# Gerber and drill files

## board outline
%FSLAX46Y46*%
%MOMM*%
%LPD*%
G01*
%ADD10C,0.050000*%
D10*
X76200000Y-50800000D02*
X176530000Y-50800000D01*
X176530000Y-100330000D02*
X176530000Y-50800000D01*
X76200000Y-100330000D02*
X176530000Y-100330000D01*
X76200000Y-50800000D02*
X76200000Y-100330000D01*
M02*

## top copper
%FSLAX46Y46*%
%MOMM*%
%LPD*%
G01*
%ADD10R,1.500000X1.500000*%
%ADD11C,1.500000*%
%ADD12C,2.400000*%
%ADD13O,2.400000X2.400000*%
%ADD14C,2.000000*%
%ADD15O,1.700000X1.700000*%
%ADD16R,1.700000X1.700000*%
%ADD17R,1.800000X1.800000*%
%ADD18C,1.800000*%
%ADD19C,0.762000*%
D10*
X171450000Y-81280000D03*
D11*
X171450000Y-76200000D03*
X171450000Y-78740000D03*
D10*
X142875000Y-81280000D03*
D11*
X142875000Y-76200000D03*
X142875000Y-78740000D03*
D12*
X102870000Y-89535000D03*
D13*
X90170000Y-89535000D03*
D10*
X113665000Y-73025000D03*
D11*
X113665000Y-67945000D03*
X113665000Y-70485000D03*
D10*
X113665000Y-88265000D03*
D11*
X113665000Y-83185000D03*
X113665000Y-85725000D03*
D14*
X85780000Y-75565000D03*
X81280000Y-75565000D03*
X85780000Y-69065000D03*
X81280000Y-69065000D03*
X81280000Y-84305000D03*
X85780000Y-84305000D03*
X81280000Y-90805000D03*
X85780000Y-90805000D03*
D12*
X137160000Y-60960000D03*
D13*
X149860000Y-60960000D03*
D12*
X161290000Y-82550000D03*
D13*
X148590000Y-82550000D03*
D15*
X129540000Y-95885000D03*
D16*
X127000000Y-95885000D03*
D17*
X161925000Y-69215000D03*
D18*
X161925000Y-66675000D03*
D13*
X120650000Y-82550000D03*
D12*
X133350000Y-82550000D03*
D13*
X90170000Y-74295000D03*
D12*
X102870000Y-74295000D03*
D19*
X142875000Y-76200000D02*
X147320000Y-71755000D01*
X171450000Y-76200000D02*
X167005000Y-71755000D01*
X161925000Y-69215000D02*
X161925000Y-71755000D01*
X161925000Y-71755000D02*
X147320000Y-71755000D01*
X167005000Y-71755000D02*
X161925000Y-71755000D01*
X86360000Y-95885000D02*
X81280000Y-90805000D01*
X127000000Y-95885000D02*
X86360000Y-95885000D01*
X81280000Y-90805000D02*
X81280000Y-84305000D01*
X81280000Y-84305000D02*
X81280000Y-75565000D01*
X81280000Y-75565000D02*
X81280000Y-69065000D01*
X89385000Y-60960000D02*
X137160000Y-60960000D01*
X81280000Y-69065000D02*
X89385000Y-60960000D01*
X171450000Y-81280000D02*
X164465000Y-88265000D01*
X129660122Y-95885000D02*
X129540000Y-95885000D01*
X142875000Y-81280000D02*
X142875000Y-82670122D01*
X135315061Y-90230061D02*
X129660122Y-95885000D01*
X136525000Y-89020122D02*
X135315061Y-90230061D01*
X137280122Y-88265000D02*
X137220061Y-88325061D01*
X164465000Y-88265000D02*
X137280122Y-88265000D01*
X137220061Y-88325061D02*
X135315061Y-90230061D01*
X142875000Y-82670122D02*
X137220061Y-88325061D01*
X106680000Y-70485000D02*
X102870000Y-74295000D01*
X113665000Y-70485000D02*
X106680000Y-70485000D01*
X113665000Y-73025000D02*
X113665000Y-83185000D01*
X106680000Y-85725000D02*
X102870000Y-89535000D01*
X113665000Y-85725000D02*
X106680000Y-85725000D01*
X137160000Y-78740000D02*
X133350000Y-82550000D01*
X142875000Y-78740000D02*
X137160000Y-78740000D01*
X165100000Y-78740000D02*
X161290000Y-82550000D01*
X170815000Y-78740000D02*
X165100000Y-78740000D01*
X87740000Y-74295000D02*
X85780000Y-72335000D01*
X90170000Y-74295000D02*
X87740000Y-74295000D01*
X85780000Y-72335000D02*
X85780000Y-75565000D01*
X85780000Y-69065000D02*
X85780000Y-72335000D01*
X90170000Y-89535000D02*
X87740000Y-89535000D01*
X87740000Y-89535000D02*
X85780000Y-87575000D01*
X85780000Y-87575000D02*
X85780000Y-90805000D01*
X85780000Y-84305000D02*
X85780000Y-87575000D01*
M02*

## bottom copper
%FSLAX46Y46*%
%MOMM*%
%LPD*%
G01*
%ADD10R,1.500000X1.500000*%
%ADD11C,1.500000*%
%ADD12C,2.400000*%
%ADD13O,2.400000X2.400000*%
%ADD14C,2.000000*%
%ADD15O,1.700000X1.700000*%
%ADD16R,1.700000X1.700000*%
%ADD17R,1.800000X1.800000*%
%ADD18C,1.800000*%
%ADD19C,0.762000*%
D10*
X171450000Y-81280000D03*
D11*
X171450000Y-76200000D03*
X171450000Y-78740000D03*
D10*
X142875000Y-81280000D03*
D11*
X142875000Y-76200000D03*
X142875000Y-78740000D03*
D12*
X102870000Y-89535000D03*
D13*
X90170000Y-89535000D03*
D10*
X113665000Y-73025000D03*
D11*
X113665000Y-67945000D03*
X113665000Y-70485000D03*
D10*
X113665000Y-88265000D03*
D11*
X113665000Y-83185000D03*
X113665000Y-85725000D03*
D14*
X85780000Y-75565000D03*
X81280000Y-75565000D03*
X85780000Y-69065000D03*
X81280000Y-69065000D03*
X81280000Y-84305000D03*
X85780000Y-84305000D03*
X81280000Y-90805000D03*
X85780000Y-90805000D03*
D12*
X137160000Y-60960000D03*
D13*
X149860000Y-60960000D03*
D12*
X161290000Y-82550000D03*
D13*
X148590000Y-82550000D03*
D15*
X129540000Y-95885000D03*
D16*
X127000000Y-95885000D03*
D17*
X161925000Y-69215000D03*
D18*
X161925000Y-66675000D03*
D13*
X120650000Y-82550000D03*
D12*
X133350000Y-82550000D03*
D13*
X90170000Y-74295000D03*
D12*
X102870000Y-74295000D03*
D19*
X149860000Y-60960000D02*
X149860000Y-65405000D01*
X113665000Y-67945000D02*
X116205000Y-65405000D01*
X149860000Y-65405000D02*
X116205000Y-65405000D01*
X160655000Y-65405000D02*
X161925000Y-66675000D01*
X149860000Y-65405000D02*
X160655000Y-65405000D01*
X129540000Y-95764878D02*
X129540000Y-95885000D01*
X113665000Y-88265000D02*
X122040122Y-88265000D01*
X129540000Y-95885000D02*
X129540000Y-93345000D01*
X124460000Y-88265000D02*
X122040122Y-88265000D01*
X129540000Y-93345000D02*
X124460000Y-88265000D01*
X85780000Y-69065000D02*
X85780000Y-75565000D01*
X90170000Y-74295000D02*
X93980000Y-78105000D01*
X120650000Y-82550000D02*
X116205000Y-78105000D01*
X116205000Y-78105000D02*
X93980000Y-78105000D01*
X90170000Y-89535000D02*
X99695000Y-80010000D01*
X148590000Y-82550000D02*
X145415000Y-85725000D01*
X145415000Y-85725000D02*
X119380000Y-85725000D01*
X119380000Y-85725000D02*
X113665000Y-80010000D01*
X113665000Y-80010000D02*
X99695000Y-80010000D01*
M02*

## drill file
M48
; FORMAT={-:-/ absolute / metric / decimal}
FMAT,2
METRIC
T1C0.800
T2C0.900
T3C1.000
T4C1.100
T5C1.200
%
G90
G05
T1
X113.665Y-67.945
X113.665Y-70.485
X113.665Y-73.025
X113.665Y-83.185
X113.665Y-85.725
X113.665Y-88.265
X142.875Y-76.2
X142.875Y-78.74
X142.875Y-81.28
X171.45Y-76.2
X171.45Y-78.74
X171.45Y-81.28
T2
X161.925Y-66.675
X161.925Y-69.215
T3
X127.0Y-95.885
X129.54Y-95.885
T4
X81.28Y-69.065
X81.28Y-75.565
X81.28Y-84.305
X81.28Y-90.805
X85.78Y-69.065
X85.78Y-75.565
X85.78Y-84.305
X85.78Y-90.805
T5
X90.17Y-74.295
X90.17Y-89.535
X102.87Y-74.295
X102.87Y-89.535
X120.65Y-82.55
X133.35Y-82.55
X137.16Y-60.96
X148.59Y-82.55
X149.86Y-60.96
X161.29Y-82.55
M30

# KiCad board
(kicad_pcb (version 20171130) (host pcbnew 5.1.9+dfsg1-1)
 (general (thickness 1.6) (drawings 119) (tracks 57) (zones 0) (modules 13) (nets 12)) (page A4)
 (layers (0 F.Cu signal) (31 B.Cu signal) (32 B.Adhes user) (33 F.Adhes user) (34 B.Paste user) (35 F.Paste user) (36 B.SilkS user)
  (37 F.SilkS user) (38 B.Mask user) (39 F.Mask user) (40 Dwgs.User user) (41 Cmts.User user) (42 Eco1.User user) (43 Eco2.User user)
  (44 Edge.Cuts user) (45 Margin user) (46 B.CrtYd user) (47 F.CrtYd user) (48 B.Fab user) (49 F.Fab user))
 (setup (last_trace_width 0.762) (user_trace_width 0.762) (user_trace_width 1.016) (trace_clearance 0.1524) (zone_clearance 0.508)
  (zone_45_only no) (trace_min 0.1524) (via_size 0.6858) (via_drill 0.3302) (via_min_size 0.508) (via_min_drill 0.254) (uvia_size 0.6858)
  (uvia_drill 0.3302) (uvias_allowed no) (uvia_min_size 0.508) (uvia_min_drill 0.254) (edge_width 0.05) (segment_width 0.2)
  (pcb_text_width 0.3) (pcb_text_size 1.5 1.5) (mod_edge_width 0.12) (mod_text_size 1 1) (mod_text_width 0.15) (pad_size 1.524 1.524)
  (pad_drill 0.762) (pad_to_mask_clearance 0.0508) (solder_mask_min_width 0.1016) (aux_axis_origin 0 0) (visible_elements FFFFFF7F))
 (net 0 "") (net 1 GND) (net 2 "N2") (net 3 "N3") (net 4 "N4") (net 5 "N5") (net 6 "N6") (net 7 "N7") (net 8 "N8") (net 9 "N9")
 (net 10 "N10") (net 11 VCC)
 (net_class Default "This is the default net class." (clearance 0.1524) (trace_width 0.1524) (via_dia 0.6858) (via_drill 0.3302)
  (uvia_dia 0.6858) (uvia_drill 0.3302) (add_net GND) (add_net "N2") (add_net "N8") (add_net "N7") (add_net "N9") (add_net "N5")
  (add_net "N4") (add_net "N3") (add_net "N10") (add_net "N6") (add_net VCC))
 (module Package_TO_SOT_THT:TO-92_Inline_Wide (layer F.Cu) (at 171.45 81.28 90)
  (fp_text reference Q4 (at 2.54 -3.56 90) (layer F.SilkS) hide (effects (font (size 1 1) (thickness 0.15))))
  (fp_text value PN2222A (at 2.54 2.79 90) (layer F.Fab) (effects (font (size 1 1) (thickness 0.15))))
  (pad 1 thru_hole rect (at 0 0 90) (size 1.5 1.5) (drill 0.8) (layers *.Cu *.Mask) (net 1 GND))
  (pad 3 thru_hole circle (at 5.08 0 90) (size 1.5 1.5) (drill 0.8) (layers *.Cu *.Mask) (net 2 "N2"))
  (pad 2 thru_hole circle (at 2.54 0 90) (size 1.5 1.5) (drill 0.8) (layers *.Cu *.Mask) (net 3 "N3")))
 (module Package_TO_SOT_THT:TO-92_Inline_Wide (layer F.Cu) (at 142.875 81.28 90)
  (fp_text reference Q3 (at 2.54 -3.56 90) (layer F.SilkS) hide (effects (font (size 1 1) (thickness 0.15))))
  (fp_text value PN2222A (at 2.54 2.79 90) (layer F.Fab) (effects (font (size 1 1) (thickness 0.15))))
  (pad 1 thru_hole rect (at 0 0 90) (size 1.5 1.5) (drill 0.8) (layers *.Cu *.Mask) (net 1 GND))
  (pad 3 thru_hole circle (at 5.08 0 90) (size 1.5 1.5) (drill 0.8) (layers *.Cu *.Mask) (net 2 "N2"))
  (pad 2 thru_hole circle (at 2.54 0 90) (size 1.5 1.5) (drill 0.8) (layers *.Cu *.Mask) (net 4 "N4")))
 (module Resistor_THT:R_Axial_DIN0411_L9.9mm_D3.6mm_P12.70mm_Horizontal (layer F.Cu) (at 102.87 89.535 180)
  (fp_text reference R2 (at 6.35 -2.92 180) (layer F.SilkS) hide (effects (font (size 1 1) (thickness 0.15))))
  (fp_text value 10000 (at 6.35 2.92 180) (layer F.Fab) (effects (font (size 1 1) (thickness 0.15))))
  (pad 1 thru_hole circle (at 0 0 180) (size 2.4 2.4) (drill 1.2) (layers *.Cu *.Mask) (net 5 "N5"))
  (pad 2 thru_hole oval (at 12.7 0 180) (size 2.4 2.4) (drill 1.2) (layers *.Cu *.Mask) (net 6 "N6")))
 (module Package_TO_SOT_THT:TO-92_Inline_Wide (layer F.Cu) (at 113.665 73.025 90)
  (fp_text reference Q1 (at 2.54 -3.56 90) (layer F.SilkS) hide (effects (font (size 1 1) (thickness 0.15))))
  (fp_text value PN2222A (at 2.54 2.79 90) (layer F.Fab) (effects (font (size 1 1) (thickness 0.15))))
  (pad 1 thru_hole rect (at 0 0 90) (size 1.5 1.5) (drill 0.8) (layers *.Cu *.Mask) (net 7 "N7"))
  (pad 3 thru_hole circle (at 5.08 0 90) (size 1.5 1.5) (drill 0.8) (layers *.Cu *.Mask) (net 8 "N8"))
  (pad 2 thru_hole circle (at 2.54 0 90) (size 1.5 1.5) (drill 0.8) (layers *.Cu *.Mask) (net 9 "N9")))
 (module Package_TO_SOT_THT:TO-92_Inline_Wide (layer F.Cu) (at 113.665 88.265 90)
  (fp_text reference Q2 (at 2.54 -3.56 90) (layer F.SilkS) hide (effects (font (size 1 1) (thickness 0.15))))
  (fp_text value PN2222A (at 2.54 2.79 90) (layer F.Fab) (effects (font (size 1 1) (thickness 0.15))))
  (pad 1 thru_hole rect (at 0 0 90) (size 1.5 1.5) (drill 0.8) (layers *.Cu *.Mask) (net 1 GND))
  (pad 3 thru_hole circle (at 5.08 0 90) (size 1.5 1.5) (drill 0.8) (layers *.Cu *.Mask) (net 7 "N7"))
  (pad 2 thru_hole circle (at 2.54 0 90) (size 1.5 1.5) (drill 0.8) (layers *.Cu *.Mask) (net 5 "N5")))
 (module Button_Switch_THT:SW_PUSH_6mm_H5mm (layer F.Cu) (at 81.28 75.565 90)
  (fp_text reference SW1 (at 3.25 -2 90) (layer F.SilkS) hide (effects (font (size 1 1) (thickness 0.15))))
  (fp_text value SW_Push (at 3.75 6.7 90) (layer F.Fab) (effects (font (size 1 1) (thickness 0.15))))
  (pad 2 thru_hole circle (at 0 4.5 180) (size 2 2) (drill 1.1) (layers *.Cu *.Mask) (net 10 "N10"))
  (pad 1 thru_hole circle (at 0 0 180) (size 2 2) (drill 1.1) (layers *.Cu *.Mask) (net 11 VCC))
  (pad 2 thru_hole circle (at 6.5 4.5 180) (size 2 2) (drill 1.1) (layers *.Cu *.Mask) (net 10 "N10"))
  (pad 1 thru_hole circle (at 6.5 0 180) (size 2 2) (drill 1.1) (layers *.Cu *.Mask) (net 11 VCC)))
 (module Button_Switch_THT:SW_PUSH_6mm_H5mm (layer F.Cu) (at 81.28 90.805 90)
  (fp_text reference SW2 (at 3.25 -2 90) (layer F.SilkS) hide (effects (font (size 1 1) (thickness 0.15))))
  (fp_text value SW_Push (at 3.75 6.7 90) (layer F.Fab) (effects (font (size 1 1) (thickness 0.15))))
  (pad 1 thru_hole circle (at 6.5 0 180) (size 2 2) (drill 1.1) (layers *.Cu *.Mask) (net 11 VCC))
  (pad 2 thru_hole circle (at 6.5 4.5 180) (size 2 2) (drill 1.1) (layers *.Cu *.Mask) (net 6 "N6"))
  (pad 1 thru_hole circle (at 0 0 180) (size 2 2) (drill 1.1) (layers *.Cu *.Mask) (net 11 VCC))
  (pad 2 thru_hole circle (at 0 4.5 180) (size 2 2) (drill 1.1) (layers *.Cu *.Mask) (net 6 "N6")))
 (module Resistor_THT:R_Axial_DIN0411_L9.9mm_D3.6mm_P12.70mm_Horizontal (layer F.Cu) (at 137.16 60.96)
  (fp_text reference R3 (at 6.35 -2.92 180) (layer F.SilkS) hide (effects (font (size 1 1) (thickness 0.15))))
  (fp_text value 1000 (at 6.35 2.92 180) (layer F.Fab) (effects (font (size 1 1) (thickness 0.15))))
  (pad 1 thru_hole circle (at 0 0) (size 2.4 2.4) (drill 1.2) (layers *.Cu *.Mask) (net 11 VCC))
  (pad 2 thru_hole oval (at 12.7 0) (size 2.4 2.4) (drill 1.2) (layers *.Cu *.Mask) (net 8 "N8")))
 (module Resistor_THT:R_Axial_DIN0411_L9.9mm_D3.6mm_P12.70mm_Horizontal (layer F.Cu) (at 161.29 82.55 180)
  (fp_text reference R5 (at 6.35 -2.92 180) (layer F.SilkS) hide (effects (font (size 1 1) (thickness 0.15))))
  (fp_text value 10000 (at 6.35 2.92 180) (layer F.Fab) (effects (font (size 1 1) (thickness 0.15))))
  (pad 1 thru_hole circle (at 0 0 180) (size 2.4 2.4) (drill 1.2) (layers *.Cu *.Mask) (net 3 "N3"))
  (pad 2 thru_hole oval (at 12.7 0 180) (size 2.4 2.4) (drill 1.2) (layers *.Cu *.Mask) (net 6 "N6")))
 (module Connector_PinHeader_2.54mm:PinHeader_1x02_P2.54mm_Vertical (layer B.Cu) (at 127 95.885 270)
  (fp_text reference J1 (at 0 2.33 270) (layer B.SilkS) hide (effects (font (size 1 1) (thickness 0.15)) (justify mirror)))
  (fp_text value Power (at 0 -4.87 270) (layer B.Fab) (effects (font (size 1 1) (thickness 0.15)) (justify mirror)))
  (pad 2 thru_hole oval (at 0 -2.54 270) (size 1.7 1.7) (drill 1) (layers *.Cu *.Mask) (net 1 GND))
  (pad 1 thru_hole rect (at 0 0 270) (size 1.7 1.7) (drill 1) (layers *.Cu *.Mask) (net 11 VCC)))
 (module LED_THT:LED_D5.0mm (layer F.Cu) (at 161.925 69.215 90)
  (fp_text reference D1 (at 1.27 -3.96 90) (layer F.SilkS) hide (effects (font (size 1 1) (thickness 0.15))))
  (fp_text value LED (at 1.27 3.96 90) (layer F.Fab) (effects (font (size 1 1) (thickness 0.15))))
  (pad 1 thru_hole rect (at 0 0 90) (size 1.8 1.8) (drill 0.9) (layers *.Cu *.Mask) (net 2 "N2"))
  (pad 2 thru_hole circle (at 2.54 0 90) (size 1.8 1.8) (drill 0.9) (layers *.Cu *.Mask) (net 8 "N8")))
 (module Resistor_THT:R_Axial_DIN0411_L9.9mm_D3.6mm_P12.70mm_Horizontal (layer F.Cu) (at 133.35 82.55 180)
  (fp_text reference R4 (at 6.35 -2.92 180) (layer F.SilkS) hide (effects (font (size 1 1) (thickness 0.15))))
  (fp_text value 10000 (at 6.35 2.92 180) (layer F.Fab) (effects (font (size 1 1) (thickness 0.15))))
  (pad 2 thru_hole oval (at 12.7 0 180) (size 2.4 2.4) (drill 1.2) (layers *.Cu *.Mask) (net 10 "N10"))
  (pad 1 thru_hole circle (at 0 0 180) (size 2.4 2.4) (drill 1.2) (layers *.Cu *.Mask) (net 4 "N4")))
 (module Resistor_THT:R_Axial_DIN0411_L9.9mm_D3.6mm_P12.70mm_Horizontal (layer F.Cu) (at 102.87 74.295 180)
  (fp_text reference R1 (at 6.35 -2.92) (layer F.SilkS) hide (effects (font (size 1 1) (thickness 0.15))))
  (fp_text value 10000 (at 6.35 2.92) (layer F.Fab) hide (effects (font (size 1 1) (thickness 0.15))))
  (pad 2 thru_hole oval (at 12.7 0 180) (size 2.4 2.4) (drill 1.2) (layers *.Cu *.Mask) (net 10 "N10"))
  (pad 1 thru_hole circle (at 0 0 180) (size 2.4 2.4) (drill 1.2) (layers *.Cu *.Mask) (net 9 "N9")))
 (gr_line (start 76.2 50.8) (end 176.53 50.8) (layer Edge.Cuts) (width 0.05))
 (gr_line (start 176.53 100.33) (end 176.53 50.8) (layer Edge.Cuts) (width 0.05))
 (gr_line (start 76.2 100.33) (end 176.53 100.33) (layer Edge.Cuts) (width 0.05))
 (gr_line (start 76.2 50.8) (end 76.2 100.33) (layer Edge.Cuts) (width 0.05))
 (segment (start 142.875 76.2) (end 147.32 71.755) (width 0.762) (layer F.Cu) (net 2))
 (segment (start 171.45 76.2) (end 167.005 71.755) (width 0.762) (layer F.Cu) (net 2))
 (segment (start 161.925 69.215) (end 161.925 71.755) (width 0.762) (layer F.Cu) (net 2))
 (segment (start 161.925 71.755) (end 147.32 71.755) (width 0.762) (layer F.Cu) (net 2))
 (segment (start 167.005 71.755) (end 161.925 71.755) (width 0.762) (layer F.Cu) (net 2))
 (segment (start 149.86 60.96) (end 149.86 65.405) (width 0.762) (layer B.Cu) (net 8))
 (segment (start 113.665 67.945) (end 116.205 65.405) (width 0.762) (layer B.Cu) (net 8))
 (segment (start 149.86 65.405) (end 116.205 65.405) (width 0.762) (layer B.Cu) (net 8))
 (segment (start 160.655 65.405) (end 161.925 66.675) (width 0.762) (layer B.Cu) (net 8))
 (segment (start 149.86 65.405) (end 160.655 65.405) (width 0.762) (layer B.Cu) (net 8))
 (segment (start 86.36 95.885) (end 81.28 90.805) (width 0.762) (layer F.Cu) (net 11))
 (segment (start 127 95.885) (end 86.36 95.885) (width 0.762) (layer F.Cu) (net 11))
 (segment (start 81.28 90.805) (end 81.28 84.305) (width 0.762) (layer F.Cu) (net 11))
 (segment (start 81.28 84.305) (end 81.28 75.565) (width 0.762) (layer F.Cu) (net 11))
 (segment (start 81.28 75.565) (end 81.28 69.065) (width 0.762) (layer F.Cu) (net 11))
 (segment (start 89.385 60.96) (end 137.16 60.96) (width 0.762) (layer F.Cu) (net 11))
 (segment (start 81.28 69.065) (end 89.385 60.96) (width 0.762) (layer F.Cu) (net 11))
 (segment (start 129.54 95.764878) (end 129.54 95.885) (width 0.762) (layer B.Cu) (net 1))
 (segment (start 113.665 88.265) (end 122.040122 88.265) (width 0.762) (layer B.Cu) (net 1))
 (segment (start 171.45 81.28) (end 164.465 88.265) (width 0.762) (layer F.Cu) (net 1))
 (segment (start 129.660122 95.885) (end 129.54 95.885) (width 0.762) (layer F.Cu) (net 1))
 (segment (start 142.875 81.28) (end 142.875 82.670122) (width 0.762) (layer F.Cu) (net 1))
 (segment (start 135.315061 90.230061) (end 129.660122 95.885) (width 0.762) (layer F.Cu) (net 1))
 (segment (start 136.525 89.020122) (end 135.315061 90.230061) (width 0.762) (layer F.Cu) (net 1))
 (segment (start 137.280122 88.265) (end 137.220061 88.325061) (width 0.762) (layer F.Cu) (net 1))
 (segment (start 164.465 88.265) (end 137.280122 88.265) (width 0.762) (layer F.Cu) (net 1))
 (segment (start 137.220061 88.325061) (end 135.315061 90.230061) (width 0.762) (layer F.Cu) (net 1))
 (segment (start 142.875 82.670122) (end 137.220061 88.325061) (width 0.762) (layer F.Cu) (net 1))
 (segment (start 129.54 95.885) (end 129.54 93.345) (width 0.762) (layer B.Cu) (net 1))
 (segment (start 124.46 88.265) (end 122.040122 88.265) (width 0.762) (layer B.Cu) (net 1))
 (segment (start 129.54 93.345) (end 124.46 88.265) (width 0.762) (layer B.Cu) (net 1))
 (segment (start 106.68 70.485) (end 102.87 74.295) (width 0.762) (layer F.Cu) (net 9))
 (segment (start 113.665 70.485) (end 106.68 70.485) (width 0.762) (layer F.Cu) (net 9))
 (segment (start 113.665 73.025) (end 113.665 83.185) (width 0.762) (layer F.Cu) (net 7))
 (segment (start 106.68 85.725) (end 102.87 89.535) (width 0.762) (layer F.Cu) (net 5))
 (segment (start 113.665 85.725) (end 106.68 85.725) (width 0.762) (layer F.Cu) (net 5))
 (segment (start 137.16 78.74) (end 133.35 82.55) (width 0.762) (layer F.Cu) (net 4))
 (segment (start 142.875 78.74) (end 137.16 78.74) (width 0.762) (layer F.Cu) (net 4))
 (segment (start 165.1 78.74) (end 161.29 82.55) (width 0.762) (layer F.Cu) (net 3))
 (segment (start 170.815 78.74) (end 165.1 78.74) (width 0.762) (layer F.Cu) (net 3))
 (segment (start 87.74 74.295) (end 85.78 72.335) (width 0.762) (layer F.Cu) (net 10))
 (segment (start 90.17 74.295) (end 87.74 74.295) (width 0.762) (layer F.Cu) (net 10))
 (segment (start 85.78 72.335) (end 85.78 75.565) (width 0.762) (layer F.Cu) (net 10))
 (segment (start 85.78 69.065) (end 85.78 72.335) (width 0.762) (layer F.Cu) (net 10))
 (segment (start 85.78 69.065) (end 85.78 75.565) (width 0.762) (layer B.Cu) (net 10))
 (segment (start 90.17 74.295) (end 93.98 78.105) (width 0.762) (layer B.Cu) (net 10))
 (segment (start 120.65 82.55) (end 116.205 78.105) (width 0.762) (layer B.Cu) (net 10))
 (segment (start 116.205 78.105) (end 93.98 78.105) (width 0.762) (layer B.Cu) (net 10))
 (segment (start 90.17 89.535) (end 87.74 89.535) (width 0.762) (layer F.Cu) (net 6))
 (segment (start 87.74 89.535) (end 85.78 87.575) (width 0.762) (layer F.Cu) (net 6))
 (segment (start 85.78 87.575) (end 85.78 90.805) (width 0.762) (layer F.Cu) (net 6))
 (segment (start 85.78 84.305) (end 85.78 87.575) (width 0.762) (layer F.Cu) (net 6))
 (segment (start 90.17 89.535) (end 99.695 80.01) (width 0.762) (layer B.Cu) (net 6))
 (segment (start 148.59 82.55) (end 145.415 85.725) (width 0.762) (layer B.Cu) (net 6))
 (segment (start 145.415 85.725) (end 119.38 85.725) (width 0.762) (layer B.Cu) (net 6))
 (segment (start 119.38 85.725) (end 113.665 80.01) (width 0.762) (layer B.Cu) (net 6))
 (segment (start 113.665 80.01) (end 99.695 80.01) (width 0.762) (layer B.Cu) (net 6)))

